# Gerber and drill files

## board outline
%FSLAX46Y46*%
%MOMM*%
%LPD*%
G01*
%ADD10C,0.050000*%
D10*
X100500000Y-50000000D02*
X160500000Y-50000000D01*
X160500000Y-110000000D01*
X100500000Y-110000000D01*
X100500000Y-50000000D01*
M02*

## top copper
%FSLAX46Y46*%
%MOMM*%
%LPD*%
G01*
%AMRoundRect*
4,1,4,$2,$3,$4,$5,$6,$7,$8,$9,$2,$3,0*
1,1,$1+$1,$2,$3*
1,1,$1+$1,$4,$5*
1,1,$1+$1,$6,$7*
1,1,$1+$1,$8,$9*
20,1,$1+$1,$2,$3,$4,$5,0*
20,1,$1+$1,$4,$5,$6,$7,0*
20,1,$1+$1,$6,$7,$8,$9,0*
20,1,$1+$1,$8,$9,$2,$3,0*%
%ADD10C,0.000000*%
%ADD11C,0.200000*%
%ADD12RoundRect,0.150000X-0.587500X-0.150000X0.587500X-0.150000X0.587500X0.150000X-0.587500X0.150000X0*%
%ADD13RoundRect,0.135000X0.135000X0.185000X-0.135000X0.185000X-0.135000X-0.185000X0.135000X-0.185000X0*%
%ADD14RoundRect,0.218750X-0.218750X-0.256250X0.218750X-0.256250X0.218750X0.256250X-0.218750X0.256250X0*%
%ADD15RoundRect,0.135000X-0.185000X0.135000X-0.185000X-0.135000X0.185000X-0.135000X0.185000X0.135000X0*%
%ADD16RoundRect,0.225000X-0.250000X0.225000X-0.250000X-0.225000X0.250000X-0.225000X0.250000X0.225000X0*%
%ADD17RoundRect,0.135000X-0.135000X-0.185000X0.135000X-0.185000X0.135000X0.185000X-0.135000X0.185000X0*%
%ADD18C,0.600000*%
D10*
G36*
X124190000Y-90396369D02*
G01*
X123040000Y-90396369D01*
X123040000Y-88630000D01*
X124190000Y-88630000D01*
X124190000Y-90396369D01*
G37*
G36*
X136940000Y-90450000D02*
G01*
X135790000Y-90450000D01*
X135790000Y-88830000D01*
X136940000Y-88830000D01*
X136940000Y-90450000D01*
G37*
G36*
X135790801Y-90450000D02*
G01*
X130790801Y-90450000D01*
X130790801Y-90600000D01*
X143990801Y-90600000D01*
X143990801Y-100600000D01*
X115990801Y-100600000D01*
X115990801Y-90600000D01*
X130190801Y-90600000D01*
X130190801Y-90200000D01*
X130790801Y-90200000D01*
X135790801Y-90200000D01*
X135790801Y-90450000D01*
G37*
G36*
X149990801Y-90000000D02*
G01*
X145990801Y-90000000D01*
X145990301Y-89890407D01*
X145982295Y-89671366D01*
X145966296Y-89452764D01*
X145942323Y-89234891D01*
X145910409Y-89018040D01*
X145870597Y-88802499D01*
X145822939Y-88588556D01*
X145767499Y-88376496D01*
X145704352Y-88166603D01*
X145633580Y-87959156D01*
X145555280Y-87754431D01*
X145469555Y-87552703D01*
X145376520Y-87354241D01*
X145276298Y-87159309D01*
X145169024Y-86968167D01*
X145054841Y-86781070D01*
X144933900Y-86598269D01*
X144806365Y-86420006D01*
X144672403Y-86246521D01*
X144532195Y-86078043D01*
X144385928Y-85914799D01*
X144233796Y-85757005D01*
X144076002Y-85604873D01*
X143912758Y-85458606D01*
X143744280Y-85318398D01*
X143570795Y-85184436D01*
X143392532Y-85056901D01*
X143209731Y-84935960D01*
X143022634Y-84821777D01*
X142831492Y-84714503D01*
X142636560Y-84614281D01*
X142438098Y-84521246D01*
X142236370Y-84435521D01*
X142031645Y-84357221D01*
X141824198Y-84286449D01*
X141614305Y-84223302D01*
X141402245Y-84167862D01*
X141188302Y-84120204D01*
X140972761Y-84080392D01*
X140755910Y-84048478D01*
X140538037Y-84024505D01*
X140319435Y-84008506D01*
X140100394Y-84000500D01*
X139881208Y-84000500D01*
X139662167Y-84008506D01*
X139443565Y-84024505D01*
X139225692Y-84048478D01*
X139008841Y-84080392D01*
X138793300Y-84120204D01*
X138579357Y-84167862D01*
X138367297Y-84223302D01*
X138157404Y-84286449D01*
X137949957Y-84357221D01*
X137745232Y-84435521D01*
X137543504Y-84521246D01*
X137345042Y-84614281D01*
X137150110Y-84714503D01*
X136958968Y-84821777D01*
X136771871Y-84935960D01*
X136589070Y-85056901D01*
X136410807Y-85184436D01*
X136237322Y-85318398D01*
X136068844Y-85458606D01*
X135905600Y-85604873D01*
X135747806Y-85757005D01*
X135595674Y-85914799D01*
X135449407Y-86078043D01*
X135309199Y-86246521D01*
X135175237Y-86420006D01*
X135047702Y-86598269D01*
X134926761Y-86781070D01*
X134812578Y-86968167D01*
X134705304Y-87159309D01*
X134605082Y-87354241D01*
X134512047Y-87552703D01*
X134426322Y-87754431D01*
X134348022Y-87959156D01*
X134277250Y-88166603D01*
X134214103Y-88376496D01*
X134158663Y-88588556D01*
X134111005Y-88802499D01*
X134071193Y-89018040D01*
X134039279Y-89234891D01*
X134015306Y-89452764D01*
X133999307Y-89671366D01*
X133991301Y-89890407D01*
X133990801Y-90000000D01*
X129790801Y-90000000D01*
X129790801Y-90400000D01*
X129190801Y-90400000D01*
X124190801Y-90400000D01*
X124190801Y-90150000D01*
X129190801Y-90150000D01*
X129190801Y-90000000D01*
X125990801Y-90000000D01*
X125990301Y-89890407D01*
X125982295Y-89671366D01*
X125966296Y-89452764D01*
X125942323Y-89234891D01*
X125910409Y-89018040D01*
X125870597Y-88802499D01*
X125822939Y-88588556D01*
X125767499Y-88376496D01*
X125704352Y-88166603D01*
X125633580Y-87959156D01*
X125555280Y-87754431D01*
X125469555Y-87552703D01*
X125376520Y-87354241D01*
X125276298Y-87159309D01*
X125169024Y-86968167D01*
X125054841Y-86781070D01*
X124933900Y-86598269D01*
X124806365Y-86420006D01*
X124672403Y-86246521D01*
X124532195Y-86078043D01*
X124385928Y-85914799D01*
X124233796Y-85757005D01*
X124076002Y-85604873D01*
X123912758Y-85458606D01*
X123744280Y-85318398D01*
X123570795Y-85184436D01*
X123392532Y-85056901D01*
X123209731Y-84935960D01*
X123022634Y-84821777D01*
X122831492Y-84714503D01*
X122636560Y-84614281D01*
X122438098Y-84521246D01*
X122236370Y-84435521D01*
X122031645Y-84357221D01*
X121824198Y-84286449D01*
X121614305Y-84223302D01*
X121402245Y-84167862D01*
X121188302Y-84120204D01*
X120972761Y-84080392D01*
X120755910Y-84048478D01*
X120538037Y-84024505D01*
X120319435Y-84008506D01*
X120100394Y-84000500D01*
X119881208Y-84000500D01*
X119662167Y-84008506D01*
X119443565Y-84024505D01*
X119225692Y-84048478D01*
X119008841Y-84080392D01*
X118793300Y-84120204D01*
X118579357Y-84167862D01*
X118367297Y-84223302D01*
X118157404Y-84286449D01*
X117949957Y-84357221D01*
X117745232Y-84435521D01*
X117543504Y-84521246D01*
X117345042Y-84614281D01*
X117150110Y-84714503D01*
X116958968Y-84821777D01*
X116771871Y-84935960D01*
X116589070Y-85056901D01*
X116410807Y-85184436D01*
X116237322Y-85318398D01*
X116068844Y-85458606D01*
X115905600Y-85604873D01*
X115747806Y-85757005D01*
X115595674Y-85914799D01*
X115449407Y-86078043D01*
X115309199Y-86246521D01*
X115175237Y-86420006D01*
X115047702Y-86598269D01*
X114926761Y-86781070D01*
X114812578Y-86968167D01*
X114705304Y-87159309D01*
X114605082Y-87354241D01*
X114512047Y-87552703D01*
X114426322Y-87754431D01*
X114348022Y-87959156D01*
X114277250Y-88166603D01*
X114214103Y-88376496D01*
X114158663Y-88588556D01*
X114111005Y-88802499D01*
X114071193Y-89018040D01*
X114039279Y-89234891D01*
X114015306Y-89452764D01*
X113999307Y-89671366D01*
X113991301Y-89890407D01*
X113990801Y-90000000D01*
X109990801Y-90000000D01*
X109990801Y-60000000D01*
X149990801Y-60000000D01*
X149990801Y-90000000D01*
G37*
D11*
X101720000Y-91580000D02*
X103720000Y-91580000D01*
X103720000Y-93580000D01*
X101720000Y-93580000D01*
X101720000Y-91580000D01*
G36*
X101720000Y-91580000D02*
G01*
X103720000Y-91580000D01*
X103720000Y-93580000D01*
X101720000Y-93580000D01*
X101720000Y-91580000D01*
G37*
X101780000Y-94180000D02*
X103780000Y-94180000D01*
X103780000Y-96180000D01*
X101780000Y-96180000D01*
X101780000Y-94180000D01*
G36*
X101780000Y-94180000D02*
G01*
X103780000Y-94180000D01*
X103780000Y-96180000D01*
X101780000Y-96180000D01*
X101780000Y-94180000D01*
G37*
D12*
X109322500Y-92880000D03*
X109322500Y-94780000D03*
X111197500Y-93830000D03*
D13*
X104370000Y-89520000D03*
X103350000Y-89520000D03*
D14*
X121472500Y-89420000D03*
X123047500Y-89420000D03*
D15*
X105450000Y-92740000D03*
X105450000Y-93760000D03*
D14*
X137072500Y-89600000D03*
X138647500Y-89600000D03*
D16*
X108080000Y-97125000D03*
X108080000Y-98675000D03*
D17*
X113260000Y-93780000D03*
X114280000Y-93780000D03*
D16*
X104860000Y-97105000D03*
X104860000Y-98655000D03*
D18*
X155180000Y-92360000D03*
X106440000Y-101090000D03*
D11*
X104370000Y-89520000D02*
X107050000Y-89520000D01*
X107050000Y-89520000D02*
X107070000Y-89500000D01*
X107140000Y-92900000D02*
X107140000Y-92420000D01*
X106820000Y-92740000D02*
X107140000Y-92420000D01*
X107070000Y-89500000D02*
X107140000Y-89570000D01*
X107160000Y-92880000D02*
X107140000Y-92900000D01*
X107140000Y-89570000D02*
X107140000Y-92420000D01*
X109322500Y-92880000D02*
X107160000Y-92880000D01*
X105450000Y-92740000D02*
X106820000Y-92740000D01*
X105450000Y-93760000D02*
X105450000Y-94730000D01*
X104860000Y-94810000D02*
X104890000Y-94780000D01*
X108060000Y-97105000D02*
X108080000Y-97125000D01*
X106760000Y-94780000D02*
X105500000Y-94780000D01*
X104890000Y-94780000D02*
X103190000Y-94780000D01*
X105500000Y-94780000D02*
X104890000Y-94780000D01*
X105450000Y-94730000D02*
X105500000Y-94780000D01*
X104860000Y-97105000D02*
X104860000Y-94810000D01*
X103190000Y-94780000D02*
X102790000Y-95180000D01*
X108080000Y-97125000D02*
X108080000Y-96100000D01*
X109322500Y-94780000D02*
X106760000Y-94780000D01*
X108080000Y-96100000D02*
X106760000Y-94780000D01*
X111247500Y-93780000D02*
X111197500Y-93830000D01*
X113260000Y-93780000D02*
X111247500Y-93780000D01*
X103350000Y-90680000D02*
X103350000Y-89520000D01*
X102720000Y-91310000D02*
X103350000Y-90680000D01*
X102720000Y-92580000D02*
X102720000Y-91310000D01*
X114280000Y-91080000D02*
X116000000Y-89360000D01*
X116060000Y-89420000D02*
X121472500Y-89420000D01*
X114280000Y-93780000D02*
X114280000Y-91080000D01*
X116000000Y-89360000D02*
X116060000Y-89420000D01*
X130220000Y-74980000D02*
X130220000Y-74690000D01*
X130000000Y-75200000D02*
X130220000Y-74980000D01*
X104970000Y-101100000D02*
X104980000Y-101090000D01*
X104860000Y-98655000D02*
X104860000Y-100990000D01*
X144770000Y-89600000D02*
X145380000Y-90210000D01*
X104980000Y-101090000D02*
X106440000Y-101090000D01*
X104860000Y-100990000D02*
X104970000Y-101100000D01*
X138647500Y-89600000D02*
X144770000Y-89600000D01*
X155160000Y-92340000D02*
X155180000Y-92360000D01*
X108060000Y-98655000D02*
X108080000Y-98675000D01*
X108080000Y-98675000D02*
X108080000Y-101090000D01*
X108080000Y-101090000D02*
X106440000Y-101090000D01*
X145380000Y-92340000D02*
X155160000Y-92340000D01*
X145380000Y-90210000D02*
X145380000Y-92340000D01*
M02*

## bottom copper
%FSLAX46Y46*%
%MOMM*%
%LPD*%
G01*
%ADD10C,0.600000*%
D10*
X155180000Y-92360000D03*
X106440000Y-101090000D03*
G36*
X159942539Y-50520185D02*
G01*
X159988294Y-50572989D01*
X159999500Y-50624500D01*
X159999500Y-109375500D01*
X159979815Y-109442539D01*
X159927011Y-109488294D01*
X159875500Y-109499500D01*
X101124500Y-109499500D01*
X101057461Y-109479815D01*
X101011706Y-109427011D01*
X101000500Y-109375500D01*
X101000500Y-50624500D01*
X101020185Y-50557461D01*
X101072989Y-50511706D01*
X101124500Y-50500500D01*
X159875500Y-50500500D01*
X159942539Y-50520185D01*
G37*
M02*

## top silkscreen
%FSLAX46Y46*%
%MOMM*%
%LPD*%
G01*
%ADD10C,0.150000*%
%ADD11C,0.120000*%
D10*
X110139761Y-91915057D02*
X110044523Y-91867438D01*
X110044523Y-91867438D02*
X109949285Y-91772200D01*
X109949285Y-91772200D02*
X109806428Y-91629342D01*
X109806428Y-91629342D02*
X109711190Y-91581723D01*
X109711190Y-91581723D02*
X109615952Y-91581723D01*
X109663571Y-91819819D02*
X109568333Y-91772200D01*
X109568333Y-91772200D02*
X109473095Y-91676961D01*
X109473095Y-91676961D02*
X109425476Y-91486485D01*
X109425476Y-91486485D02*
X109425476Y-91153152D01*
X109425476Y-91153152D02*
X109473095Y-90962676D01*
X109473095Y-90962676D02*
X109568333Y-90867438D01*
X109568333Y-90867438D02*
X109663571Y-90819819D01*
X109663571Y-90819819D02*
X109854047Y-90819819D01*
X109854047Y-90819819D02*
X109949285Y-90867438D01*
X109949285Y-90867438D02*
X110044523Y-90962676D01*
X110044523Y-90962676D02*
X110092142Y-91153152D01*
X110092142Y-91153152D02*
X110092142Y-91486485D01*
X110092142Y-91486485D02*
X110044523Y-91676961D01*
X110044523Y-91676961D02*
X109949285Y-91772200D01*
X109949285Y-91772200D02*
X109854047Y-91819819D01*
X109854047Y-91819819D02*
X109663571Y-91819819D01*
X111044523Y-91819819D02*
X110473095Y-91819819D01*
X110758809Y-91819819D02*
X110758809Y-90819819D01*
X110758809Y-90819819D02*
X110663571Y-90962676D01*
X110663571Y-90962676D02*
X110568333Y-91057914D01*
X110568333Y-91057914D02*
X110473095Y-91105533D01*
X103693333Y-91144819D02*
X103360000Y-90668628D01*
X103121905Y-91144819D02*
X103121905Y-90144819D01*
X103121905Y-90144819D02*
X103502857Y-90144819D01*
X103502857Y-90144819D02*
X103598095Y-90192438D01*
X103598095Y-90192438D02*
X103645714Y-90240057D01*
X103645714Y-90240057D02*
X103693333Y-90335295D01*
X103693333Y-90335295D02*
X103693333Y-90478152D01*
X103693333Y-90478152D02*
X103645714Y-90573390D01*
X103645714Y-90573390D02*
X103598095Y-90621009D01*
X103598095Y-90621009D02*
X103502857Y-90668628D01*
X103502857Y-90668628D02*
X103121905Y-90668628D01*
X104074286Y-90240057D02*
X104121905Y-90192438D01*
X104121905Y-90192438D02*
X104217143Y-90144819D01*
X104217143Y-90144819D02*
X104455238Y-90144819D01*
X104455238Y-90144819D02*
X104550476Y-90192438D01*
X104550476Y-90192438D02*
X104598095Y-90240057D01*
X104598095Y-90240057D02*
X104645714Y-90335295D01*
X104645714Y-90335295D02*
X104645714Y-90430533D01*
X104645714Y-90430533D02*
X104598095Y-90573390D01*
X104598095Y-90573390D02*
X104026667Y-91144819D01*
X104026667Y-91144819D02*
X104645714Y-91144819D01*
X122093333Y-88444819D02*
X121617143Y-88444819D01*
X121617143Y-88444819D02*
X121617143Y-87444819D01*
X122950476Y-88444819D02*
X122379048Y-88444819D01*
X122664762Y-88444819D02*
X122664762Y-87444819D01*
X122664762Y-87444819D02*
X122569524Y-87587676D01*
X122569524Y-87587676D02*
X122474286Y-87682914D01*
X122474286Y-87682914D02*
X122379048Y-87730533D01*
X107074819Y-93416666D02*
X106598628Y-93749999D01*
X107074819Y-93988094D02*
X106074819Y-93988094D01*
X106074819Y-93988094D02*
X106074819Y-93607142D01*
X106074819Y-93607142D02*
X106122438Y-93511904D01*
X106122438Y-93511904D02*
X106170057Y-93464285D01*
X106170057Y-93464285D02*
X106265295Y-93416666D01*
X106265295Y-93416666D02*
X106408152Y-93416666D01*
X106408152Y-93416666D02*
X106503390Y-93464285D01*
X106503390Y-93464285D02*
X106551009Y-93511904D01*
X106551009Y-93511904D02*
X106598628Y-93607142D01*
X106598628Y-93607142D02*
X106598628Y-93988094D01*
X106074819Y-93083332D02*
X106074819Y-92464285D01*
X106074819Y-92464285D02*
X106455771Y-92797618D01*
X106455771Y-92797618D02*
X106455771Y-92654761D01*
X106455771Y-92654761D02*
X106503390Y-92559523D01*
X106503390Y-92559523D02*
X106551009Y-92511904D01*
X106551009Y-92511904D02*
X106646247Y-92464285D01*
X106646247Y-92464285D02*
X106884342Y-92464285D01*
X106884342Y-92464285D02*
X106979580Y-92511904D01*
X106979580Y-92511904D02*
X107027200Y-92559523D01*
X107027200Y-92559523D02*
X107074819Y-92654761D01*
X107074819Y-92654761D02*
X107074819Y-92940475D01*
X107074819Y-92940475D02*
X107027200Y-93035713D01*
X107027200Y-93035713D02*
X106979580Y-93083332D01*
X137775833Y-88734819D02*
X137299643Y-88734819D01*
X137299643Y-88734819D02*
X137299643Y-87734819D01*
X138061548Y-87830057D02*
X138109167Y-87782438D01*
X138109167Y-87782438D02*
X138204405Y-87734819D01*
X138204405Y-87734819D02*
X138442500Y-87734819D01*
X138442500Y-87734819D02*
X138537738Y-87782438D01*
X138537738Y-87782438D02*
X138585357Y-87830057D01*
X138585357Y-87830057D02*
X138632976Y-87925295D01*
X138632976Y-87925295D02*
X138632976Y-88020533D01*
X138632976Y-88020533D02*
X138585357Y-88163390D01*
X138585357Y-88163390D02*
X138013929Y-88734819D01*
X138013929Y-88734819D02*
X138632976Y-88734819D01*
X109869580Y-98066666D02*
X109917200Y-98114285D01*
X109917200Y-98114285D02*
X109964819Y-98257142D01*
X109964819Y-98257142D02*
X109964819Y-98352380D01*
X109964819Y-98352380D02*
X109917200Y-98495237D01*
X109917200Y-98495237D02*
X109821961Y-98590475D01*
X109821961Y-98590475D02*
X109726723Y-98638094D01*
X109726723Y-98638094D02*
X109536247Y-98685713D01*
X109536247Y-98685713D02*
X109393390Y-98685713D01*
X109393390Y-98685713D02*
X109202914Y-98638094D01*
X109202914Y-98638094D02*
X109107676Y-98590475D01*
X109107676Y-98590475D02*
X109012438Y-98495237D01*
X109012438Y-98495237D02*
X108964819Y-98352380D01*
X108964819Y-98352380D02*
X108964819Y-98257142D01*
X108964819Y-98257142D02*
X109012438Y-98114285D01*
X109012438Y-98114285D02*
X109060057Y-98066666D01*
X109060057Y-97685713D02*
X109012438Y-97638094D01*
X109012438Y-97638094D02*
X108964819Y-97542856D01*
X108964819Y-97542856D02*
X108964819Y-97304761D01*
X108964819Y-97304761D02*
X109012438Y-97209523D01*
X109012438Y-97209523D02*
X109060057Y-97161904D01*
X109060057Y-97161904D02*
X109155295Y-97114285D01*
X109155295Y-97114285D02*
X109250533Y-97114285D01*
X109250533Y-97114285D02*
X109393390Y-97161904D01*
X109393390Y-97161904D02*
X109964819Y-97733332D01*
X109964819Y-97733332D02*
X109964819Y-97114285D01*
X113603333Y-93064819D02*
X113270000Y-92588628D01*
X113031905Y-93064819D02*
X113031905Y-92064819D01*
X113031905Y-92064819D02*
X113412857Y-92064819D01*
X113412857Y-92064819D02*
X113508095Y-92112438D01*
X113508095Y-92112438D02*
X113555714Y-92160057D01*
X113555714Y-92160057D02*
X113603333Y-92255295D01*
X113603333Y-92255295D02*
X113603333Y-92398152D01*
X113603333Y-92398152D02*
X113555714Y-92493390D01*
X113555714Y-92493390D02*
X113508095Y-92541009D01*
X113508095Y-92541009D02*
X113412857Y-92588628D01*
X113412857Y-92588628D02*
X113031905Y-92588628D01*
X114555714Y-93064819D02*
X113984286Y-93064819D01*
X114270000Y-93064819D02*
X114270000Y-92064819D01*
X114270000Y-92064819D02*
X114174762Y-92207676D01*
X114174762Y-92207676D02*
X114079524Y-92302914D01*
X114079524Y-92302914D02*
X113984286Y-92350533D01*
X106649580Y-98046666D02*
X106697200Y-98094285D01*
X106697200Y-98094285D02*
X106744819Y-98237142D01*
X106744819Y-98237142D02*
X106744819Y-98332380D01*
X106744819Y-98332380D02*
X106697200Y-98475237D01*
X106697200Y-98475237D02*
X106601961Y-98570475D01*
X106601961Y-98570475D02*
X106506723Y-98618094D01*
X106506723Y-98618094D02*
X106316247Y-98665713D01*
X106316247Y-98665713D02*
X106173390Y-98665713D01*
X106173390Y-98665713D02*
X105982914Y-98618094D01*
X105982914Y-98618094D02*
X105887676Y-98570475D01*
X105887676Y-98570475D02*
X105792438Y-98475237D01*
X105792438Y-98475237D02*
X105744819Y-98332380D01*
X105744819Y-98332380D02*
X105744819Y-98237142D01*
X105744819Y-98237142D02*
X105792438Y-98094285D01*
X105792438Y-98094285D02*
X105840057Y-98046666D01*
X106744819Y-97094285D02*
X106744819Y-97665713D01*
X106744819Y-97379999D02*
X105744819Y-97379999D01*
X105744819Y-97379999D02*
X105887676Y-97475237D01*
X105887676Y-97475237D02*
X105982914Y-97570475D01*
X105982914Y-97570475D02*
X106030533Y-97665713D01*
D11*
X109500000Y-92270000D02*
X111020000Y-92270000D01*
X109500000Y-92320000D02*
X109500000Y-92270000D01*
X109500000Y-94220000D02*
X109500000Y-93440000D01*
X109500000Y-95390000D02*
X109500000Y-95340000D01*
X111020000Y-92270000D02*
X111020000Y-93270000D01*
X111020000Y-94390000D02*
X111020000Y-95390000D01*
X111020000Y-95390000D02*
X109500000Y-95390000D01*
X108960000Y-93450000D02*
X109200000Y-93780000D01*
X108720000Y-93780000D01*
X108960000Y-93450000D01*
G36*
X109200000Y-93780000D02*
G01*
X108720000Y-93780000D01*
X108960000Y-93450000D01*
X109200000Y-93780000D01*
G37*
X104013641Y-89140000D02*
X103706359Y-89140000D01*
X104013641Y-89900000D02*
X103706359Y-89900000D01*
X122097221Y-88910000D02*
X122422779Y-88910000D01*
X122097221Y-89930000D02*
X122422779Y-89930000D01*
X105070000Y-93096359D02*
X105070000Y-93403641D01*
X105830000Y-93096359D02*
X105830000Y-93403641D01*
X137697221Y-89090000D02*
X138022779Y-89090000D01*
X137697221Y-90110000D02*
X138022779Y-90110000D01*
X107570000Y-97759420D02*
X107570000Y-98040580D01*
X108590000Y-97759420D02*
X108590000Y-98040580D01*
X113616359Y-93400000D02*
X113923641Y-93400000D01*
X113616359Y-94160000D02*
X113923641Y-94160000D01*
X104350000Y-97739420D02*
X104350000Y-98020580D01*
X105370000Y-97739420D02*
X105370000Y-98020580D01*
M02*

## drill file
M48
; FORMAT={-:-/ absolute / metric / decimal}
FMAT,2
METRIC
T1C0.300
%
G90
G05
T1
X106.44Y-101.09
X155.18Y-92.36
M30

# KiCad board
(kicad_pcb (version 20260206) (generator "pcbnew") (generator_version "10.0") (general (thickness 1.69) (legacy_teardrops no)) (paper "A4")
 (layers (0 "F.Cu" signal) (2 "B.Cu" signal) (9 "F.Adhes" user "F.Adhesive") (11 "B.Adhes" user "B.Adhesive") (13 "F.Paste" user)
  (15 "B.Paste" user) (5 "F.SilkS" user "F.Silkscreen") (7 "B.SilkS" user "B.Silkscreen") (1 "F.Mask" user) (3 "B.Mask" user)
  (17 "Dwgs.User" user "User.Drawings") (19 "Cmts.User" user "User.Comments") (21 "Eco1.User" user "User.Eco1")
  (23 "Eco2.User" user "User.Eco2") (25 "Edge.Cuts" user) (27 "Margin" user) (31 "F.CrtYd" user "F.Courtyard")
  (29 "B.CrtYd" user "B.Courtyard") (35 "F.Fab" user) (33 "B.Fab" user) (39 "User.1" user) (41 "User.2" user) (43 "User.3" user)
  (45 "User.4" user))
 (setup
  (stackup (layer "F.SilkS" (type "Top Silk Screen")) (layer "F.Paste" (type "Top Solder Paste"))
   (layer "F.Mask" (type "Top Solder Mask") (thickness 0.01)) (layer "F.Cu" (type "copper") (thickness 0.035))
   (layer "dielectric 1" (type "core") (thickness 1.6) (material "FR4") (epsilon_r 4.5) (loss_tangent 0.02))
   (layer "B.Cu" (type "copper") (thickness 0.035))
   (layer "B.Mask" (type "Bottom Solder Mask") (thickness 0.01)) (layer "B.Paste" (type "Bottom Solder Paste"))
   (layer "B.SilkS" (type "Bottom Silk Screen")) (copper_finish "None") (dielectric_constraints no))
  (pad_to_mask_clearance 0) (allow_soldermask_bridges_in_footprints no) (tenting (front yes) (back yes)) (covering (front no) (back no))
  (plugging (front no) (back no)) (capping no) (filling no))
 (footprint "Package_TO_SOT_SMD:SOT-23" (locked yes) (layer "F.Cu") (at 110.26 93.83)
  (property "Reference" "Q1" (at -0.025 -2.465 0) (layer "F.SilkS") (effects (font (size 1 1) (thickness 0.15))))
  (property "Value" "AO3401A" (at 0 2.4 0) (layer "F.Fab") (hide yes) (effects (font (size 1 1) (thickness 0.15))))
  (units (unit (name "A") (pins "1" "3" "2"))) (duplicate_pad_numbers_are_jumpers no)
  (fp_line (start -0.76 -1.56) (end 0.76 -1.56) (stroke (width 0.12) (type solid)) (layer "F.SilkS"))
  (fp_line (start -0.76 -1.51) (end -0.76 -1.56) (stroke (width 0.12) (type solid)) (layer "F.SilkS"))
  (fp_line (start -0.76 0.39) (end -0.76 -0.39) (stroke (width 0.12) (type solid)) (layer "F.SilkS"))
  (fp_line (start -0.76 1.56) (end -0.76 1.51) (stroke (width 0.12) (type solid)) (layer "F.SilkS"))
  (fp_line (start 0.76 -1.56) (end 0.76 -0.56) (stroke (width 0.12) (type solid)) (layer "F.SilkS"))
  (fp_line (start 0.76 0.56) (end 0.76 1.56) (stroke (width 0.12) (type solid)) (layer "F.SilkS"))
  (fp_line (start 0.76 1.56) (end -0.76 1.56) (stroke (width 0.12) (type solid)) (layer "F.SilkS"))
  (fp_poly (pts (xy -1.3 -0.38) (xy -1.06 -0.05) (xy -1.54 -0.05)) (stroke (width 0.12) (type solid)) (fill yes) (layer "F.SilkS"))
  (pad "1" smd roundrect (at -0.9375 -0.95) (size 1.475 0.6) (layers "F.Cu" "F.Mask" "F.Paste") (roundrect_rratio 0.25) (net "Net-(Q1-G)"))
  (pad "2" smd roundrect (at -0.9375 0.95) (size 1.475 0.6) (layers "F.Cu" "F.Mask" "F.Paste") (roundrect_rratio 0.25) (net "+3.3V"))
  (pad "3" smd roundrect (at 0.9375 0) (size 1.475 0.6) (layers "F.Cu" "F.Mask" "F.Paste") (roundrect_rratio 0.25) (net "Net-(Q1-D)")))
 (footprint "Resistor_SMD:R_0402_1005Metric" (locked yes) (layer "F.Cu") (at 103.86 89.52 180)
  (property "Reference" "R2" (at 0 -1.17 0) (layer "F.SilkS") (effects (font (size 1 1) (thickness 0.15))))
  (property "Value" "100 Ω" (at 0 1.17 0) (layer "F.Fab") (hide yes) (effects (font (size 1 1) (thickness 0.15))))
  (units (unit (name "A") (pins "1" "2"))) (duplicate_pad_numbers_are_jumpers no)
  (fp_line (start -0.153641 0.38) (end 0.153641 0.38) (stroke (width 0.12) (type solid)) (layer "F.SilkS"))
  (fp_line (start -0.153641 -0.38) (end 0.153641 -0.38) (stroke (width 0.12) (type solid)) (layer "F.SilkS"))
  (pad "1" smd roundrect (at -0.51 0 180) (size 0.54 0.64) (layers "F.Cu" "F.Mask" "F.Paste") (roundrect_rratio 0.25) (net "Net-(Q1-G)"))
  (pad "2" smd roundrect (at 0.51 0 180) (size 0.54 0.64) (layers "F.Cu" "F.Mask" "F.Paste") (roundrect_rratio 0.25) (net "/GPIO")))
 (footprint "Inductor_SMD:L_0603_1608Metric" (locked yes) (layer "F.Cu") (at 122.26 89.42)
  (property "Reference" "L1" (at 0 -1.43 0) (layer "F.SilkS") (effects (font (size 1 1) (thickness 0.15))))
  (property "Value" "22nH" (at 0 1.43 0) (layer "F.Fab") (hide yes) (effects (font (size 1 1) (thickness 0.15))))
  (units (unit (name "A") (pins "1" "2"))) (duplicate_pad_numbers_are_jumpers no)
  (fp_line (start -0.162779 -0.51) (end 0.162779 -0.51) (stroke (width 0.12) (type solid)) (layer "F.SilkS"))
  (fp_line (start -0.162779 0.51) (end 0.162779 0.51) (stroke (width 0.12) (type solid)) (layer "F.SilkS"))
  (pad "1" smd roundrect (at -0.7875 0) (size 0.875 0.95) (layers "F.Cu" "F.Mask" "F.Paste") (roundrect_rratio 0.25) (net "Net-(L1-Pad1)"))
  (pad "2" smd roundrect (at 0.7875 0) (size 0.875 0.95) (layers "F.Cu" "F.Mask" "F.Paste") (roundrect_rratio 0.25)
   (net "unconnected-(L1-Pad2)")))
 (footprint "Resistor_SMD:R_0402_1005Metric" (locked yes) (layer "F.Cu") (at 105.45 93.25 -90)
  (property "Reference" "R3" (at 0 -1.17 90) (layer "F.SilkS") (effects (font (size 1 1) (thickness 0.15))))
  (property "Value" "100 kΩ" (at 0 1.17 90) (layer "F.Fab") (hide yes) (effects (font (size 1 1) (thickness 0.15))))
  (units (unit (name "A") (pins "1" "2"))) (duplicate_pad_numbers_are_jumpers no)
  (fp_line (start -0.153641 0.38) (end 0.153641 0.38) (stroke (width 0.12) (type solid)) (layer "F.SilkS"))
  (fp_line (start -0.153641 -0.38) (end 0.153641 -0.38) (stroke (width 0.12) (type solid)) (layer "F.SilkS"))
  (pad "1" smd roundrect (at -0.51 0 270) (size 0.54 0.64) (layers "F.Cu" "F.Mask" "F.Paste") (roundrect_rratio 0.25) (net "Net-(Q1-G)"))
  (pad "2" smd roundrect (at 0.51 0 270) (size 0.54 0.64) (layers "F.Cu" "F.Mask" "F.Paste") (roundrect_rratio 0.25) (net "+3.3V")))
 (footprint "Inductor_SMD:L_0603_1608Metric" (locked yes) (layer "F.Cu") (at 137.86 89.6)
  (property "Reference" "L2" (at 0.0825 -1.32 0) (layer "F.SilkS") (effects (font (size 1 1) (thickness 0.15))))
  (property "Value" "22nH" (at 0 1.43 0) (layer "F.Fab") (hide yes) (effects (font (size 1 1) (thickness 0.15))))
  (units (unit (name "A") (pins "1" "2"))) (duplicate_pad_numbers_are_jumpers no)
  (fp_line (start -0.162779 -0.51) (end 0.162779 -0.51) (stroke (width 0.12) (type solid)) (layer "F.SilkS"))
  (fp_line (start -0.162779 0.51) (end 0.162779 0.51) (stroke (width 0.12) (type solid)) (layer "F.SilkS"))
  (pad "1" smd roundrect (at -0.7875 0) (size 0.875 0.95) (layers "F.Cu" "F.Mask" "F.Paste") (roundrect_rratio 0.25)
   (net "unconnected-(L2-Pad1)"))
  (pad "2" smd roundrect (at 0.7875 0) (size 0.875 0.95) (layers "F.Cu" "F.Mask" "F.Paste") (roundrect_rratio 0.25) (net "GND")))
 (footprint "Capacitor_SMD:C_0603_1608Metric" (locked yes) (layer "F.Cu") (at 108.08 97.9 -90)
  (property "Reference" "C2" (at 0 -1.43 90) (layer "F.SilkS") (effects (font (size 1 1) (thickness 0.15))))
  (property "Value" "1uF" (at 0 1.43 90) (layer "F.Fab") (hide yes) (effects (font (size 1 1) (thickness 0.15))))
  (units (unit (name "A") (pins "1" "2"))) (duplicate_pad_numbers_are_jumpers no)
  (fp_line (start -0.14058 0.51) (end 0.14058 0.51) (stroke (width 0.12) (type solid)) (layer "F.SilkS"))
  (fp_line (start -0.14058 -0.51) (end 0.14058 -0.51) (stroke (width 0.12) (type solid)) (layer "F.SilkS"))
  (pad "1" smd roundrect (at -0.775 0 270) (size 0.9 0.95) (layers "F.Cu" "F.Mask" "F.Paste") (roundrect_rratio 0.25) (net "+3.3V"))
  (pad "2" smd roundrect (at 0.775 0 270) (size 0.9 0.95) (layers "F.Cu" "F.Mask" "F.Paste") (roundrect_rratio 0.25) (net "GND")))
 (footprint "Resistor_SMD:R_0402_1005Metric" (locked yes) (layer "F.Cu") (at 113.77 93.78)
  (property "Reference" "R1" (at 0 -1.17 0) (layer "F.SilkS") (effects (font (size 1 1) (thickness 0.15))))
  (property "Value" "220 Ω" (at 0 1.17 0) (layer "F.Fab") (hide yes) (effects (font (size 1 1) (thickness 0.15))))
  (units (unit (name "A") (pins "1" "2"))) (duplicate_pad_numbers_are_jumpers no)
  (fp_line (start -0.153641 -0.38) (end 0.153641 -0.38) (stroke (width 0.12) (type solid)) (layer "F.SilkS"))
  (fp_line (start -0.153641 0.38) (end 0.153641 0.38) (stroke (width 0.12) (type solid)) (layer "F.SilkS"))
  (pad "1" smd roundrect (at -0.51 0) (size 0.54 0.64) (layers "F.Cu" "F.Mask" "F.Paste") (roundrect_rratio 0.25) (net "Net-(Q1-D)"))
  (pad "2" smd roundrect (at 0.51 0) (size 0.54 0.64) (layers "F.Cu" "F.Mask" "F.Paste") (roundrect_rratio 0.25) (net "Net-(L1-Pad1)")))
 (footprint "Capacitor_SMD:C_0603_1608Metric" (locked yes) (layer "F.Cu") (at 104.86 97.88 -90)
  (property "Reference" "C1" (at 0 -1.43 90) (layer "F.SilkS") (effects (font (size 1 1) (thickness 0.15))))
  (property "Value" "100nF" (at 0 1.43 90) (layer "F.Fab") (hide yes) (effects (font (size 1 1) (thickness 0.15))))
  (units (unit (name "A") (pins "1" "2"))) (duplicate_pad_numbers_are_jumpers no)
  (fp_line (start -0.14058 0.51) (end 0.14058 0.51) (stroke (width 0.12) (type solid)) (layer "F.SilkS"))
  (fp_line (start -0.14058 -0.51) (end 0.14058 -0.51) (stroke (width 0.12) (type solid)) (layer "F.SilkS"))
  (pad "1" smd roundrect (at -0.775 0 270) (size 0.9 0.95) (layers "F.Cu" "F.Mask" "F.Paste") (roundrect_rratio 0.25) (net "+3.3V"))
  (pad "2" smd roundrect (at 0.775 0 270) (size 0.9 0.95) (layers "F.Cu" "F.Mask" "F.Paste") (roundrect_rratio 0.25) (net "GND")))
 (gr_poly
  (pts (xy 123.04 88.63) (xy 124.19 88.63) (xy 124.19 90.396369) (xy 123.04 90.396369)) (stroke (width 0) (type solid)) (fill yes)
  (locked yes) (layer "F.Cu") (net "unconnected-(L1-Pad2)"))
 (gr_poly
  (pts (xy 135.79 88.83) (xy 136.94 88.83) (xy 136.94 90.45) (xy 135.79 90.45)) (stroke (width 0) (type solid)) (fill yes) (locked yes)
  (layer "F.Cu") (net "unconnected-(L2-Pad1)"))
 (gr_poly
  (pts (xy 143.990801 90.6) (xy 143.990801 100.6) (xy 115.990801 100.6) (xy 115.990801 90.6) (xy 130.190801 90.6) (xy 130.190801 90.2)
   (xy 130.790801 90.2) (xy 135.790801 90.2) (xy 135.790801 90.45) (xy 130.790801 90.45) (xy 130.790801 90.6))
  (stroke (width 0) (type solid)) (fill yes) (locked yes) (layer "F.Cu") (net "unconnected-(L2-Pad1)"))
 (gr_poly
  (pts (xy 109.990801 60) (xy 149.990801 60) (xy 149.990801 90) (xy 145.990801 90) (xy 145.990301 89.890407) (xy 145.982295 89.671366)
   (xy 145.966296 89.452764) (xy 145.942323 89.234891) (xy 145.910409 89.01804) (xy 145.870597 88.802499) (xy 145.822939 88.588556)
   (xy 145.767499 88.376496) (xy 145.704352 88.166603) (xy 145.63358 87.959156) (xy 145.55528 87.754431) (xy 145.469555 87.552703)
   (xy 145.37652 87.354241) (xy 145.276298 87.159309) (xy 145.169024 86.968167) (xy 145.054841 86.78107) (xy 144.9339 86.598269)
   (xy 144.806365 86.420006) (xy 144.672403 86.246521) (xy 144.532195 86.078043) (xy 144.385928 85.914799) (xy 144.233796 85.757005)
   (xy 144.076002 85.604873) (xy 143.912758 85.458606) (xy 143.74428 85.318398) (xy 143.570795 85.184436) (xy 143.392532 85.056901)
   (xy 143.209731 84.93596) (xy 143.022634 84.821777) (xy 142.831492 84.714503) (xy 142.63656 84.614281) (xy 142.438098 84.521246)
   (xy 142.23637 84.435521) (xy 142.031645 84.357221) (xy 141.824198 84.286449) (xy 141.614305 84.223302) (xy 141.402245 84.167862)
   (xy 141.188302 84.120204) (xy 140.972761 84.080392) (xy 140.75591 84.048478) (xy 140.538037 84.024505) (xy 140.319435 84.008506)
   (xy 140.100394 84.0005) (xy 139.881208 84.0005) (xy 139.662167 84.008506) (xy 139.443565 84.024505) (xy 139.225692 84.048478)
   (xy 139.008841 84.080392) (xy 138.7933 84.120204) (xy 138.579357 84.167862) (xy 138.367297 84.223302) (xy 138.157404 84.286449)
   (xy 137.949957 84.357221) (xy 137.745232 84.435521) (xy 137.543504 84.521246) (xy 137.345042 84.614281) (xy 137.15011 84.714503)
   (xy 136.958968 84.821777) (xy 136.771871 84.93596) (xy 136.58907 85.056901) (xy 136.410807 85.184436) (xy 136.237322 85.318398)
   (xy 136.068844 85.458606) (xy 135.9056 85.604873) (xy 135.747806 85.757005) (xy 135.595674 85.914799) (xy 135.449407 86.078043)
   (xy 135.309199 86.246521) (xy 135.175237 86.420006) (xy 135.047702 86.598269) (xy 134.926761 86.78107) (xy 134.812578 86.968167)
   (xy 134.705304 87.159309) (xy 134.605082 87.354241) (xy 134.512047 87.552703) (xy 134.426322 87.754431) (xy 134.348022 87.959156)
   (xy 134.27725 88.166603) (xy 134.214103 88.376496) (xy 134.158663 88.588556) (xy 134.111005 88.802499) (xy 134.071193 89.01804)
   (xy 134.039279 89.234891) (xy 134.015306 89.452764) (xy 133.999307 89.671366) (xy 133.991301 89.890407) (xy 133.990801 90)
   (xy 129.790801 90) (xy 129.790801 90.4) (xy 129.190801 90.4) (xy 124.190801 90.4) (xy 124.190801 90.15) (xy 129.190801 90.15)
   (xy 129.190801 90) (xy 125.990801 90) (xy 125.990301 89.890407) (xy 125.982295 89.671366) (xy 125.966296 89.452764)
   (xy 125.942323 89.234891) (xy 125.910409 89.01804) (xy 125.870597 88.802499) (xy 125.822939 88.588556) (xy 125.767499 88.376496)
   (xy 125.704352 88.166603) (xy 125.63358 87.959156) (xy 125.55528 87.754431) (xy 125.469555 87.552703) (xy 125.37652 87.354241)
   (xy 125.276298 87.159309) (xy 125.169024 86.968167) (xy 125.054841 86.78107) (xy 124.9339 86.598269) (xy 124.806365 86.420006)
   (xy 124.672403 86.246521) (xy 124.532195 86.078043) (xy 124.385928 85.914799) (xy 124.233796 85.757005) (xy 124.076002 85.604873)
   (xy 123.912758 85.458606) (xy 123.74428 85.318398) (xy 123.570795 85.184436) (xy 123.392532 85.056901) (xy 123.209731 84.93596)
   (xy 123.022634 84.821777) (xy 122.831492 84.714503) (xy 122.63656 84.614281) (xy 122.438098 84.521246) (xy 122.23637 84.435521)
   (xy 122.031645 84.357221) (xy 121.824198 84.286449) (xy 121.614305 84.223302) (xy 121.402245 84.167862) (xy 121.188302 84.120204)
   (xy 120.972761 84.080392) (xy 120.75591 84.048478) (xy 120.538037 84.024505) (xy 120.319435 84.008506) (xy 120.100394 84.0005)
   (xy 119.881208 84.0005) (xy 119.662167 84.008506) (xy 119.443565 84.024505) (xy 119.225692 84.048478) (xy 119.008841 84.080392)
   (xy 118.7933 84.120204) (xy 118.579357 84.167862) (xy 118.367297 84.223302) (xy 118.157404 84.286449) (xy 117.949957 84.357221)
   (xy 117.745232 84.435521) (xy 117.543504 84.521246) (xy 117.345042 84.614281) (xy 117.15011 84.714503) (xy 116.958968 84.821777)
   (xy 116.771871 84.93596) (xy 116.58907 85.056901) (xy 116.410807 85.184436) (xy 116.237322 85.318398) (xy 116.068844 85.458606)
   (xy 115.9056 85.604873) (xy 115.747806 85.757005) (xy 115.595674 85.914799) (xy 115.449407 86.078043) (xy 115.309199 86.246521)
   (xy 115.175237 86.420006) (xy 115.047702 86.598269) (xy 114.926761 86.78107) (xy 114.812578 86.968167) (xy 114.705304 87.159309)
   (xy 114.605082 87.354241) (xy 114.512047 87.552703) (xy 114.426322 87.754431) (xy 114.348022 87.959156) (xy 114.27725 88.166603)
   (xy 114.214103 88.376496) (xy 114.158663 88.588556) (xy 114.111005 88.802499) (xy 114.071193 89.01804) (xy 114.039279 89.234891)
   (xy 114.015306 89.452764) (xy 113.999307 89.671366) (xy 113.991301 89.890407) (xy 113.990801 90) (xy 109.990801 90))
  (stroke (width 0) (type solid)) (fill yes) (locked yes) (layer "F.Cu") (net "unconnected-(L1-Pad2)"))
 (gr_rect (start 101.72 91.58) (end 103.72 93.58) (stroke (width 0.2) (type default)) (fill yes) (locked yes) (layer "F.Cu") (net "/GPIO"))
 (gr_rect (start 101.78 94.18) (end 103.78 96.18) (stroke (width 0.2) (type default)) (fill yes) (locked yes) (layer "F.Cu") (net "+3.3V"))
 (gr_rect (start 100.5 50) (end 160.5 110) (stroke (width 0.05) (type default)) (fill no) (locked yes) (layer "Edge.Cuts"))
 (segment (start 104.37 89.52) (end 107.05 89.52) (width 0.2) (locked yes) (layer "F.Cu") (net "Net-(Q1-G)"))
 (segment (start 107.05 89.52) (end 107.07 89.5) (width 0.2) (locked yes) (layer "F.Cu") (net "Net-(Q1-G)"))
 (segment (start 107.14 92.9) (end 107.14 92.42) (width 0.2) (locked yes) (layer "F.Cu") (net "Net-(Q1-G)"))
 (segment (start 106.82 92.74) (end 107.14 92.42) (width 0.2) (locked yes) (layer "F.Cu") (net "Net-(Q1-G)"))
 (segment (start 107.07 89.5) (end 107.14 89.57) (width 0.2) (locked yes) (layer "F.Cu") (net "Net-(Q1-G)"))
 (segment (start 107.16 92.88) (end 107.14 92.9) (width 0.2) (locked yes) (layer "F.Cu") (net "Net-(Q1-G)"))
 (segment (start 107.14 89.57) (end 107.14 92.42) (width 0.2) (locked yes) (layer "F.Cu") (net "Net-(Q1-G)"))
 (segment (start 109.3225 92.88) (end 107.16 92.88) (width 0.2) (locked yes) (layer "F.Cu") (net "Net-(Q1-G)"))
 (segment (start 105.45 92.74) (end 106.82 92.74) (width 0.2) (locked yes) (layer "F.Cu") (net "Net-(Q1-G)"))
 (segment (start 105.45 93.76) (end 105.45 94.73) (width 0.2) (locked yes) (layer "F.Cu") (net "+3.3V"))
 (segment (start 104.86 94.81) (end 104.89 94.78) (width 0.2) (locked yes) (layer "F.Cu") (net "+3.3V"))
 (segment (start 108.06 97.105) (end 108.08 97.125) (width 0.2) (locked yes) (layer "F.Cu") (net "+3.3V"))
 (segment (start 106.76 94.78) (end 105.5 94.78) (width 0.2) (locked yes) (layer "F.Cu") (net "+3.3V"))
 (segment (start 104.89 94.78) (end 103.19 94.78) (width 0.2) (locked yes) (layer "F.Cu") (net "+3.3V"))
 (segment (start 105.5 94.78) (end 104.89 94.78) (width 0.2) (locked yes) (layer "F.Cu") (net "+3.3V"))
 (segment (start 105.45 94.73) (end 105.5 94.78) (width 0.2) (locked yes) (layer "F.Cu") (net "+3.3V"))
 (segment (start 104.86 97.105) (end 104.86 94.81) (width 0.2) (locked yes) (layer "F.Cu") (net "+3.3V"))
 (segment (start 103.19 94.78) (end 102.79 95.18) (width 0.2) (locked yes) (layer "F.Cu") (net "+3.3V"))
 (segment (start 108.08 97.125) (end 108.08 96.1) (width 0.2) (locked yes) (layer "F.Cu") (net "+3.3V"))
 (segment (start 109.3225 94.78) (end 106.76 94.78) (width 0.2) (locked yes) (layer "F.Cu") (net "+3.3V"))
 (segment (start 108.08 96.1) (end 106.76 94.78) (width 0.2) (locked yes) (layer "F.Cu") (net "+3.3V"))
 (segment (start 111.2475 93.78) (end 111.1975 93.83) (width 0.2) (locked yes) (layer "F.Cu") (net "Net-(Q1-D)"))
 (segment (start 113.26 93.78) (end 111.2475 93.78) (width 0.2) (locked yes) (layer "F.Cu") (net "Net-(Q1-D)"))
 (segment (start 103.35 90.68) (end 103.35 89.52) (width 0.2) (locked yes) (layer "F.Cu") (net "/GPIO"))
 (segment (start 102.72 91.31) (end 103.35 90.68) (width 0.2) (locked yes) (layer "F.Cu") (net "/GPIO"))
 (segment (start 102.72 92.58) (end 102.72 91.31) (width 0.2) (locked yes) (layer "F.Cu") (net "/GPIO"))
 (segment (start 114.28 91.08) (end 116 89.36) (width 0.2) (locked yes) (layer "F.Cu") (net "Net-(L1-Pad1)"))
 (segment (start 116.06 89.42) (end 121.4725 89.42) (width 0.2) (locked yes) (layer "F.Cu") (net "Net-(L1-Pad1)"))
 (segment (start 114.28 93.78) (end 114.28 91.08) (width 0.2) (locked yes) (layer "F.Cu") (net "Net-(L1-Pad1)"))
 (segment (start 116 89.36) (end 116.06 89.42) (width 0.2) (locked yes) (layer "F.Cu") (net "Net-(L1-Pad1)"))
 (segment (start 130.22 74.98) (end 130.22 74.69) (width 0.2) (locked yes) (layer "F.Cu") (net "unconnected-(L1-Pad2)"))
 (segment (start 130 75.2) (end 130.22 74.98) (width 0.2) (locked yes) (layer "F.Cu") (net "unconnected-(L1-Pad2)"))
 (segment (start 104.97 101.1) (end 104.98 101.09) (width 0.2) (locked yes) (layer "F.Cu") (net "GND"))
 (segment (start 104.86 98.655) (end 104.86 100.99) (width 0.2) (locked yes) (layer "F.Cu") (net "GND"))
 (segment (start 144.77 89.6) (end 145.38 90.21) (width 0.2) (locked yes) (layer "F.Cu") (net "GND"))
 (segment (start 104.98 101.09) (end 106.44 101.09) (width 0.2) (locked yes) (layer "F.Cu") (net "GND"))
 (segment (start 104.86 100.99) (end 104.97 101.1) (width 0.2) (locked yes) (layer "F.Cu") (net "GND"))
 (segment (start 138.6475 89.6) (end 144.77 89.6) (width 0.2) (locked yes) (layer "F.Cu") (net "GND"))
 (segment (start 155.16 92.34) (end 155.18 92.36) (width 0.2) (locked yes) (layer "F.Cu") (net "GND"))
 (segment (start 108.06 98.655) (end 108.08 98.675) (width 0.2) (locked yes) (layer "F.Cu") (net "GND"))
 (segment (start 108.08 98.675) (end 108.08 101.09) (width 0.2) (locked yes) (layer "F.Cu") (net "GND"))
 (segment (start 108.08 101.09) (end 106.44 101.09) (width 0.2) (locked yes) (layer "F.Cu") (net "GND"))
 (segment (start 145.38 92.34) (end 155.16 92.34) (width 0.2) (locked yes) (layer "F.Cu") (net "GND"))
 (segment (start 145.38 90.21) (end 145.38 92.34) (width 0.2) (locked yes) (layer "F.Cu") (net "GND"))
 (via (at 155.18 92.36) (size 0.6) (drill 0.3) (layers "F.Cu" "B.Cu") (locked yes) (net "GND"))
 (via (at 106.44 101.09) (size 0.6) (drill 0.3) (layers "F.Cu" "B.Cu") (locked yes) (tenting (front no) (back no)) (capping no)
  (covering (front no) (back no)) (plugging (front no) (back no)) (filling no) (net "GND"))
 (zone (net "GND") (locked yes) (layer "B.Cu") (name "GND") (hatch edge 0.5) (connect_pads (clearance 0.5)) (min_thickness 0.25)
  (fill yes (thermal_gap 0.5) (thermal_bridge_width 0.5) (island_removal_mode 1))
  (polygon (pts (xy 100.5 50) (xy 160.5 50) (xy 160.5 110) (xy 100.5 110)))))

